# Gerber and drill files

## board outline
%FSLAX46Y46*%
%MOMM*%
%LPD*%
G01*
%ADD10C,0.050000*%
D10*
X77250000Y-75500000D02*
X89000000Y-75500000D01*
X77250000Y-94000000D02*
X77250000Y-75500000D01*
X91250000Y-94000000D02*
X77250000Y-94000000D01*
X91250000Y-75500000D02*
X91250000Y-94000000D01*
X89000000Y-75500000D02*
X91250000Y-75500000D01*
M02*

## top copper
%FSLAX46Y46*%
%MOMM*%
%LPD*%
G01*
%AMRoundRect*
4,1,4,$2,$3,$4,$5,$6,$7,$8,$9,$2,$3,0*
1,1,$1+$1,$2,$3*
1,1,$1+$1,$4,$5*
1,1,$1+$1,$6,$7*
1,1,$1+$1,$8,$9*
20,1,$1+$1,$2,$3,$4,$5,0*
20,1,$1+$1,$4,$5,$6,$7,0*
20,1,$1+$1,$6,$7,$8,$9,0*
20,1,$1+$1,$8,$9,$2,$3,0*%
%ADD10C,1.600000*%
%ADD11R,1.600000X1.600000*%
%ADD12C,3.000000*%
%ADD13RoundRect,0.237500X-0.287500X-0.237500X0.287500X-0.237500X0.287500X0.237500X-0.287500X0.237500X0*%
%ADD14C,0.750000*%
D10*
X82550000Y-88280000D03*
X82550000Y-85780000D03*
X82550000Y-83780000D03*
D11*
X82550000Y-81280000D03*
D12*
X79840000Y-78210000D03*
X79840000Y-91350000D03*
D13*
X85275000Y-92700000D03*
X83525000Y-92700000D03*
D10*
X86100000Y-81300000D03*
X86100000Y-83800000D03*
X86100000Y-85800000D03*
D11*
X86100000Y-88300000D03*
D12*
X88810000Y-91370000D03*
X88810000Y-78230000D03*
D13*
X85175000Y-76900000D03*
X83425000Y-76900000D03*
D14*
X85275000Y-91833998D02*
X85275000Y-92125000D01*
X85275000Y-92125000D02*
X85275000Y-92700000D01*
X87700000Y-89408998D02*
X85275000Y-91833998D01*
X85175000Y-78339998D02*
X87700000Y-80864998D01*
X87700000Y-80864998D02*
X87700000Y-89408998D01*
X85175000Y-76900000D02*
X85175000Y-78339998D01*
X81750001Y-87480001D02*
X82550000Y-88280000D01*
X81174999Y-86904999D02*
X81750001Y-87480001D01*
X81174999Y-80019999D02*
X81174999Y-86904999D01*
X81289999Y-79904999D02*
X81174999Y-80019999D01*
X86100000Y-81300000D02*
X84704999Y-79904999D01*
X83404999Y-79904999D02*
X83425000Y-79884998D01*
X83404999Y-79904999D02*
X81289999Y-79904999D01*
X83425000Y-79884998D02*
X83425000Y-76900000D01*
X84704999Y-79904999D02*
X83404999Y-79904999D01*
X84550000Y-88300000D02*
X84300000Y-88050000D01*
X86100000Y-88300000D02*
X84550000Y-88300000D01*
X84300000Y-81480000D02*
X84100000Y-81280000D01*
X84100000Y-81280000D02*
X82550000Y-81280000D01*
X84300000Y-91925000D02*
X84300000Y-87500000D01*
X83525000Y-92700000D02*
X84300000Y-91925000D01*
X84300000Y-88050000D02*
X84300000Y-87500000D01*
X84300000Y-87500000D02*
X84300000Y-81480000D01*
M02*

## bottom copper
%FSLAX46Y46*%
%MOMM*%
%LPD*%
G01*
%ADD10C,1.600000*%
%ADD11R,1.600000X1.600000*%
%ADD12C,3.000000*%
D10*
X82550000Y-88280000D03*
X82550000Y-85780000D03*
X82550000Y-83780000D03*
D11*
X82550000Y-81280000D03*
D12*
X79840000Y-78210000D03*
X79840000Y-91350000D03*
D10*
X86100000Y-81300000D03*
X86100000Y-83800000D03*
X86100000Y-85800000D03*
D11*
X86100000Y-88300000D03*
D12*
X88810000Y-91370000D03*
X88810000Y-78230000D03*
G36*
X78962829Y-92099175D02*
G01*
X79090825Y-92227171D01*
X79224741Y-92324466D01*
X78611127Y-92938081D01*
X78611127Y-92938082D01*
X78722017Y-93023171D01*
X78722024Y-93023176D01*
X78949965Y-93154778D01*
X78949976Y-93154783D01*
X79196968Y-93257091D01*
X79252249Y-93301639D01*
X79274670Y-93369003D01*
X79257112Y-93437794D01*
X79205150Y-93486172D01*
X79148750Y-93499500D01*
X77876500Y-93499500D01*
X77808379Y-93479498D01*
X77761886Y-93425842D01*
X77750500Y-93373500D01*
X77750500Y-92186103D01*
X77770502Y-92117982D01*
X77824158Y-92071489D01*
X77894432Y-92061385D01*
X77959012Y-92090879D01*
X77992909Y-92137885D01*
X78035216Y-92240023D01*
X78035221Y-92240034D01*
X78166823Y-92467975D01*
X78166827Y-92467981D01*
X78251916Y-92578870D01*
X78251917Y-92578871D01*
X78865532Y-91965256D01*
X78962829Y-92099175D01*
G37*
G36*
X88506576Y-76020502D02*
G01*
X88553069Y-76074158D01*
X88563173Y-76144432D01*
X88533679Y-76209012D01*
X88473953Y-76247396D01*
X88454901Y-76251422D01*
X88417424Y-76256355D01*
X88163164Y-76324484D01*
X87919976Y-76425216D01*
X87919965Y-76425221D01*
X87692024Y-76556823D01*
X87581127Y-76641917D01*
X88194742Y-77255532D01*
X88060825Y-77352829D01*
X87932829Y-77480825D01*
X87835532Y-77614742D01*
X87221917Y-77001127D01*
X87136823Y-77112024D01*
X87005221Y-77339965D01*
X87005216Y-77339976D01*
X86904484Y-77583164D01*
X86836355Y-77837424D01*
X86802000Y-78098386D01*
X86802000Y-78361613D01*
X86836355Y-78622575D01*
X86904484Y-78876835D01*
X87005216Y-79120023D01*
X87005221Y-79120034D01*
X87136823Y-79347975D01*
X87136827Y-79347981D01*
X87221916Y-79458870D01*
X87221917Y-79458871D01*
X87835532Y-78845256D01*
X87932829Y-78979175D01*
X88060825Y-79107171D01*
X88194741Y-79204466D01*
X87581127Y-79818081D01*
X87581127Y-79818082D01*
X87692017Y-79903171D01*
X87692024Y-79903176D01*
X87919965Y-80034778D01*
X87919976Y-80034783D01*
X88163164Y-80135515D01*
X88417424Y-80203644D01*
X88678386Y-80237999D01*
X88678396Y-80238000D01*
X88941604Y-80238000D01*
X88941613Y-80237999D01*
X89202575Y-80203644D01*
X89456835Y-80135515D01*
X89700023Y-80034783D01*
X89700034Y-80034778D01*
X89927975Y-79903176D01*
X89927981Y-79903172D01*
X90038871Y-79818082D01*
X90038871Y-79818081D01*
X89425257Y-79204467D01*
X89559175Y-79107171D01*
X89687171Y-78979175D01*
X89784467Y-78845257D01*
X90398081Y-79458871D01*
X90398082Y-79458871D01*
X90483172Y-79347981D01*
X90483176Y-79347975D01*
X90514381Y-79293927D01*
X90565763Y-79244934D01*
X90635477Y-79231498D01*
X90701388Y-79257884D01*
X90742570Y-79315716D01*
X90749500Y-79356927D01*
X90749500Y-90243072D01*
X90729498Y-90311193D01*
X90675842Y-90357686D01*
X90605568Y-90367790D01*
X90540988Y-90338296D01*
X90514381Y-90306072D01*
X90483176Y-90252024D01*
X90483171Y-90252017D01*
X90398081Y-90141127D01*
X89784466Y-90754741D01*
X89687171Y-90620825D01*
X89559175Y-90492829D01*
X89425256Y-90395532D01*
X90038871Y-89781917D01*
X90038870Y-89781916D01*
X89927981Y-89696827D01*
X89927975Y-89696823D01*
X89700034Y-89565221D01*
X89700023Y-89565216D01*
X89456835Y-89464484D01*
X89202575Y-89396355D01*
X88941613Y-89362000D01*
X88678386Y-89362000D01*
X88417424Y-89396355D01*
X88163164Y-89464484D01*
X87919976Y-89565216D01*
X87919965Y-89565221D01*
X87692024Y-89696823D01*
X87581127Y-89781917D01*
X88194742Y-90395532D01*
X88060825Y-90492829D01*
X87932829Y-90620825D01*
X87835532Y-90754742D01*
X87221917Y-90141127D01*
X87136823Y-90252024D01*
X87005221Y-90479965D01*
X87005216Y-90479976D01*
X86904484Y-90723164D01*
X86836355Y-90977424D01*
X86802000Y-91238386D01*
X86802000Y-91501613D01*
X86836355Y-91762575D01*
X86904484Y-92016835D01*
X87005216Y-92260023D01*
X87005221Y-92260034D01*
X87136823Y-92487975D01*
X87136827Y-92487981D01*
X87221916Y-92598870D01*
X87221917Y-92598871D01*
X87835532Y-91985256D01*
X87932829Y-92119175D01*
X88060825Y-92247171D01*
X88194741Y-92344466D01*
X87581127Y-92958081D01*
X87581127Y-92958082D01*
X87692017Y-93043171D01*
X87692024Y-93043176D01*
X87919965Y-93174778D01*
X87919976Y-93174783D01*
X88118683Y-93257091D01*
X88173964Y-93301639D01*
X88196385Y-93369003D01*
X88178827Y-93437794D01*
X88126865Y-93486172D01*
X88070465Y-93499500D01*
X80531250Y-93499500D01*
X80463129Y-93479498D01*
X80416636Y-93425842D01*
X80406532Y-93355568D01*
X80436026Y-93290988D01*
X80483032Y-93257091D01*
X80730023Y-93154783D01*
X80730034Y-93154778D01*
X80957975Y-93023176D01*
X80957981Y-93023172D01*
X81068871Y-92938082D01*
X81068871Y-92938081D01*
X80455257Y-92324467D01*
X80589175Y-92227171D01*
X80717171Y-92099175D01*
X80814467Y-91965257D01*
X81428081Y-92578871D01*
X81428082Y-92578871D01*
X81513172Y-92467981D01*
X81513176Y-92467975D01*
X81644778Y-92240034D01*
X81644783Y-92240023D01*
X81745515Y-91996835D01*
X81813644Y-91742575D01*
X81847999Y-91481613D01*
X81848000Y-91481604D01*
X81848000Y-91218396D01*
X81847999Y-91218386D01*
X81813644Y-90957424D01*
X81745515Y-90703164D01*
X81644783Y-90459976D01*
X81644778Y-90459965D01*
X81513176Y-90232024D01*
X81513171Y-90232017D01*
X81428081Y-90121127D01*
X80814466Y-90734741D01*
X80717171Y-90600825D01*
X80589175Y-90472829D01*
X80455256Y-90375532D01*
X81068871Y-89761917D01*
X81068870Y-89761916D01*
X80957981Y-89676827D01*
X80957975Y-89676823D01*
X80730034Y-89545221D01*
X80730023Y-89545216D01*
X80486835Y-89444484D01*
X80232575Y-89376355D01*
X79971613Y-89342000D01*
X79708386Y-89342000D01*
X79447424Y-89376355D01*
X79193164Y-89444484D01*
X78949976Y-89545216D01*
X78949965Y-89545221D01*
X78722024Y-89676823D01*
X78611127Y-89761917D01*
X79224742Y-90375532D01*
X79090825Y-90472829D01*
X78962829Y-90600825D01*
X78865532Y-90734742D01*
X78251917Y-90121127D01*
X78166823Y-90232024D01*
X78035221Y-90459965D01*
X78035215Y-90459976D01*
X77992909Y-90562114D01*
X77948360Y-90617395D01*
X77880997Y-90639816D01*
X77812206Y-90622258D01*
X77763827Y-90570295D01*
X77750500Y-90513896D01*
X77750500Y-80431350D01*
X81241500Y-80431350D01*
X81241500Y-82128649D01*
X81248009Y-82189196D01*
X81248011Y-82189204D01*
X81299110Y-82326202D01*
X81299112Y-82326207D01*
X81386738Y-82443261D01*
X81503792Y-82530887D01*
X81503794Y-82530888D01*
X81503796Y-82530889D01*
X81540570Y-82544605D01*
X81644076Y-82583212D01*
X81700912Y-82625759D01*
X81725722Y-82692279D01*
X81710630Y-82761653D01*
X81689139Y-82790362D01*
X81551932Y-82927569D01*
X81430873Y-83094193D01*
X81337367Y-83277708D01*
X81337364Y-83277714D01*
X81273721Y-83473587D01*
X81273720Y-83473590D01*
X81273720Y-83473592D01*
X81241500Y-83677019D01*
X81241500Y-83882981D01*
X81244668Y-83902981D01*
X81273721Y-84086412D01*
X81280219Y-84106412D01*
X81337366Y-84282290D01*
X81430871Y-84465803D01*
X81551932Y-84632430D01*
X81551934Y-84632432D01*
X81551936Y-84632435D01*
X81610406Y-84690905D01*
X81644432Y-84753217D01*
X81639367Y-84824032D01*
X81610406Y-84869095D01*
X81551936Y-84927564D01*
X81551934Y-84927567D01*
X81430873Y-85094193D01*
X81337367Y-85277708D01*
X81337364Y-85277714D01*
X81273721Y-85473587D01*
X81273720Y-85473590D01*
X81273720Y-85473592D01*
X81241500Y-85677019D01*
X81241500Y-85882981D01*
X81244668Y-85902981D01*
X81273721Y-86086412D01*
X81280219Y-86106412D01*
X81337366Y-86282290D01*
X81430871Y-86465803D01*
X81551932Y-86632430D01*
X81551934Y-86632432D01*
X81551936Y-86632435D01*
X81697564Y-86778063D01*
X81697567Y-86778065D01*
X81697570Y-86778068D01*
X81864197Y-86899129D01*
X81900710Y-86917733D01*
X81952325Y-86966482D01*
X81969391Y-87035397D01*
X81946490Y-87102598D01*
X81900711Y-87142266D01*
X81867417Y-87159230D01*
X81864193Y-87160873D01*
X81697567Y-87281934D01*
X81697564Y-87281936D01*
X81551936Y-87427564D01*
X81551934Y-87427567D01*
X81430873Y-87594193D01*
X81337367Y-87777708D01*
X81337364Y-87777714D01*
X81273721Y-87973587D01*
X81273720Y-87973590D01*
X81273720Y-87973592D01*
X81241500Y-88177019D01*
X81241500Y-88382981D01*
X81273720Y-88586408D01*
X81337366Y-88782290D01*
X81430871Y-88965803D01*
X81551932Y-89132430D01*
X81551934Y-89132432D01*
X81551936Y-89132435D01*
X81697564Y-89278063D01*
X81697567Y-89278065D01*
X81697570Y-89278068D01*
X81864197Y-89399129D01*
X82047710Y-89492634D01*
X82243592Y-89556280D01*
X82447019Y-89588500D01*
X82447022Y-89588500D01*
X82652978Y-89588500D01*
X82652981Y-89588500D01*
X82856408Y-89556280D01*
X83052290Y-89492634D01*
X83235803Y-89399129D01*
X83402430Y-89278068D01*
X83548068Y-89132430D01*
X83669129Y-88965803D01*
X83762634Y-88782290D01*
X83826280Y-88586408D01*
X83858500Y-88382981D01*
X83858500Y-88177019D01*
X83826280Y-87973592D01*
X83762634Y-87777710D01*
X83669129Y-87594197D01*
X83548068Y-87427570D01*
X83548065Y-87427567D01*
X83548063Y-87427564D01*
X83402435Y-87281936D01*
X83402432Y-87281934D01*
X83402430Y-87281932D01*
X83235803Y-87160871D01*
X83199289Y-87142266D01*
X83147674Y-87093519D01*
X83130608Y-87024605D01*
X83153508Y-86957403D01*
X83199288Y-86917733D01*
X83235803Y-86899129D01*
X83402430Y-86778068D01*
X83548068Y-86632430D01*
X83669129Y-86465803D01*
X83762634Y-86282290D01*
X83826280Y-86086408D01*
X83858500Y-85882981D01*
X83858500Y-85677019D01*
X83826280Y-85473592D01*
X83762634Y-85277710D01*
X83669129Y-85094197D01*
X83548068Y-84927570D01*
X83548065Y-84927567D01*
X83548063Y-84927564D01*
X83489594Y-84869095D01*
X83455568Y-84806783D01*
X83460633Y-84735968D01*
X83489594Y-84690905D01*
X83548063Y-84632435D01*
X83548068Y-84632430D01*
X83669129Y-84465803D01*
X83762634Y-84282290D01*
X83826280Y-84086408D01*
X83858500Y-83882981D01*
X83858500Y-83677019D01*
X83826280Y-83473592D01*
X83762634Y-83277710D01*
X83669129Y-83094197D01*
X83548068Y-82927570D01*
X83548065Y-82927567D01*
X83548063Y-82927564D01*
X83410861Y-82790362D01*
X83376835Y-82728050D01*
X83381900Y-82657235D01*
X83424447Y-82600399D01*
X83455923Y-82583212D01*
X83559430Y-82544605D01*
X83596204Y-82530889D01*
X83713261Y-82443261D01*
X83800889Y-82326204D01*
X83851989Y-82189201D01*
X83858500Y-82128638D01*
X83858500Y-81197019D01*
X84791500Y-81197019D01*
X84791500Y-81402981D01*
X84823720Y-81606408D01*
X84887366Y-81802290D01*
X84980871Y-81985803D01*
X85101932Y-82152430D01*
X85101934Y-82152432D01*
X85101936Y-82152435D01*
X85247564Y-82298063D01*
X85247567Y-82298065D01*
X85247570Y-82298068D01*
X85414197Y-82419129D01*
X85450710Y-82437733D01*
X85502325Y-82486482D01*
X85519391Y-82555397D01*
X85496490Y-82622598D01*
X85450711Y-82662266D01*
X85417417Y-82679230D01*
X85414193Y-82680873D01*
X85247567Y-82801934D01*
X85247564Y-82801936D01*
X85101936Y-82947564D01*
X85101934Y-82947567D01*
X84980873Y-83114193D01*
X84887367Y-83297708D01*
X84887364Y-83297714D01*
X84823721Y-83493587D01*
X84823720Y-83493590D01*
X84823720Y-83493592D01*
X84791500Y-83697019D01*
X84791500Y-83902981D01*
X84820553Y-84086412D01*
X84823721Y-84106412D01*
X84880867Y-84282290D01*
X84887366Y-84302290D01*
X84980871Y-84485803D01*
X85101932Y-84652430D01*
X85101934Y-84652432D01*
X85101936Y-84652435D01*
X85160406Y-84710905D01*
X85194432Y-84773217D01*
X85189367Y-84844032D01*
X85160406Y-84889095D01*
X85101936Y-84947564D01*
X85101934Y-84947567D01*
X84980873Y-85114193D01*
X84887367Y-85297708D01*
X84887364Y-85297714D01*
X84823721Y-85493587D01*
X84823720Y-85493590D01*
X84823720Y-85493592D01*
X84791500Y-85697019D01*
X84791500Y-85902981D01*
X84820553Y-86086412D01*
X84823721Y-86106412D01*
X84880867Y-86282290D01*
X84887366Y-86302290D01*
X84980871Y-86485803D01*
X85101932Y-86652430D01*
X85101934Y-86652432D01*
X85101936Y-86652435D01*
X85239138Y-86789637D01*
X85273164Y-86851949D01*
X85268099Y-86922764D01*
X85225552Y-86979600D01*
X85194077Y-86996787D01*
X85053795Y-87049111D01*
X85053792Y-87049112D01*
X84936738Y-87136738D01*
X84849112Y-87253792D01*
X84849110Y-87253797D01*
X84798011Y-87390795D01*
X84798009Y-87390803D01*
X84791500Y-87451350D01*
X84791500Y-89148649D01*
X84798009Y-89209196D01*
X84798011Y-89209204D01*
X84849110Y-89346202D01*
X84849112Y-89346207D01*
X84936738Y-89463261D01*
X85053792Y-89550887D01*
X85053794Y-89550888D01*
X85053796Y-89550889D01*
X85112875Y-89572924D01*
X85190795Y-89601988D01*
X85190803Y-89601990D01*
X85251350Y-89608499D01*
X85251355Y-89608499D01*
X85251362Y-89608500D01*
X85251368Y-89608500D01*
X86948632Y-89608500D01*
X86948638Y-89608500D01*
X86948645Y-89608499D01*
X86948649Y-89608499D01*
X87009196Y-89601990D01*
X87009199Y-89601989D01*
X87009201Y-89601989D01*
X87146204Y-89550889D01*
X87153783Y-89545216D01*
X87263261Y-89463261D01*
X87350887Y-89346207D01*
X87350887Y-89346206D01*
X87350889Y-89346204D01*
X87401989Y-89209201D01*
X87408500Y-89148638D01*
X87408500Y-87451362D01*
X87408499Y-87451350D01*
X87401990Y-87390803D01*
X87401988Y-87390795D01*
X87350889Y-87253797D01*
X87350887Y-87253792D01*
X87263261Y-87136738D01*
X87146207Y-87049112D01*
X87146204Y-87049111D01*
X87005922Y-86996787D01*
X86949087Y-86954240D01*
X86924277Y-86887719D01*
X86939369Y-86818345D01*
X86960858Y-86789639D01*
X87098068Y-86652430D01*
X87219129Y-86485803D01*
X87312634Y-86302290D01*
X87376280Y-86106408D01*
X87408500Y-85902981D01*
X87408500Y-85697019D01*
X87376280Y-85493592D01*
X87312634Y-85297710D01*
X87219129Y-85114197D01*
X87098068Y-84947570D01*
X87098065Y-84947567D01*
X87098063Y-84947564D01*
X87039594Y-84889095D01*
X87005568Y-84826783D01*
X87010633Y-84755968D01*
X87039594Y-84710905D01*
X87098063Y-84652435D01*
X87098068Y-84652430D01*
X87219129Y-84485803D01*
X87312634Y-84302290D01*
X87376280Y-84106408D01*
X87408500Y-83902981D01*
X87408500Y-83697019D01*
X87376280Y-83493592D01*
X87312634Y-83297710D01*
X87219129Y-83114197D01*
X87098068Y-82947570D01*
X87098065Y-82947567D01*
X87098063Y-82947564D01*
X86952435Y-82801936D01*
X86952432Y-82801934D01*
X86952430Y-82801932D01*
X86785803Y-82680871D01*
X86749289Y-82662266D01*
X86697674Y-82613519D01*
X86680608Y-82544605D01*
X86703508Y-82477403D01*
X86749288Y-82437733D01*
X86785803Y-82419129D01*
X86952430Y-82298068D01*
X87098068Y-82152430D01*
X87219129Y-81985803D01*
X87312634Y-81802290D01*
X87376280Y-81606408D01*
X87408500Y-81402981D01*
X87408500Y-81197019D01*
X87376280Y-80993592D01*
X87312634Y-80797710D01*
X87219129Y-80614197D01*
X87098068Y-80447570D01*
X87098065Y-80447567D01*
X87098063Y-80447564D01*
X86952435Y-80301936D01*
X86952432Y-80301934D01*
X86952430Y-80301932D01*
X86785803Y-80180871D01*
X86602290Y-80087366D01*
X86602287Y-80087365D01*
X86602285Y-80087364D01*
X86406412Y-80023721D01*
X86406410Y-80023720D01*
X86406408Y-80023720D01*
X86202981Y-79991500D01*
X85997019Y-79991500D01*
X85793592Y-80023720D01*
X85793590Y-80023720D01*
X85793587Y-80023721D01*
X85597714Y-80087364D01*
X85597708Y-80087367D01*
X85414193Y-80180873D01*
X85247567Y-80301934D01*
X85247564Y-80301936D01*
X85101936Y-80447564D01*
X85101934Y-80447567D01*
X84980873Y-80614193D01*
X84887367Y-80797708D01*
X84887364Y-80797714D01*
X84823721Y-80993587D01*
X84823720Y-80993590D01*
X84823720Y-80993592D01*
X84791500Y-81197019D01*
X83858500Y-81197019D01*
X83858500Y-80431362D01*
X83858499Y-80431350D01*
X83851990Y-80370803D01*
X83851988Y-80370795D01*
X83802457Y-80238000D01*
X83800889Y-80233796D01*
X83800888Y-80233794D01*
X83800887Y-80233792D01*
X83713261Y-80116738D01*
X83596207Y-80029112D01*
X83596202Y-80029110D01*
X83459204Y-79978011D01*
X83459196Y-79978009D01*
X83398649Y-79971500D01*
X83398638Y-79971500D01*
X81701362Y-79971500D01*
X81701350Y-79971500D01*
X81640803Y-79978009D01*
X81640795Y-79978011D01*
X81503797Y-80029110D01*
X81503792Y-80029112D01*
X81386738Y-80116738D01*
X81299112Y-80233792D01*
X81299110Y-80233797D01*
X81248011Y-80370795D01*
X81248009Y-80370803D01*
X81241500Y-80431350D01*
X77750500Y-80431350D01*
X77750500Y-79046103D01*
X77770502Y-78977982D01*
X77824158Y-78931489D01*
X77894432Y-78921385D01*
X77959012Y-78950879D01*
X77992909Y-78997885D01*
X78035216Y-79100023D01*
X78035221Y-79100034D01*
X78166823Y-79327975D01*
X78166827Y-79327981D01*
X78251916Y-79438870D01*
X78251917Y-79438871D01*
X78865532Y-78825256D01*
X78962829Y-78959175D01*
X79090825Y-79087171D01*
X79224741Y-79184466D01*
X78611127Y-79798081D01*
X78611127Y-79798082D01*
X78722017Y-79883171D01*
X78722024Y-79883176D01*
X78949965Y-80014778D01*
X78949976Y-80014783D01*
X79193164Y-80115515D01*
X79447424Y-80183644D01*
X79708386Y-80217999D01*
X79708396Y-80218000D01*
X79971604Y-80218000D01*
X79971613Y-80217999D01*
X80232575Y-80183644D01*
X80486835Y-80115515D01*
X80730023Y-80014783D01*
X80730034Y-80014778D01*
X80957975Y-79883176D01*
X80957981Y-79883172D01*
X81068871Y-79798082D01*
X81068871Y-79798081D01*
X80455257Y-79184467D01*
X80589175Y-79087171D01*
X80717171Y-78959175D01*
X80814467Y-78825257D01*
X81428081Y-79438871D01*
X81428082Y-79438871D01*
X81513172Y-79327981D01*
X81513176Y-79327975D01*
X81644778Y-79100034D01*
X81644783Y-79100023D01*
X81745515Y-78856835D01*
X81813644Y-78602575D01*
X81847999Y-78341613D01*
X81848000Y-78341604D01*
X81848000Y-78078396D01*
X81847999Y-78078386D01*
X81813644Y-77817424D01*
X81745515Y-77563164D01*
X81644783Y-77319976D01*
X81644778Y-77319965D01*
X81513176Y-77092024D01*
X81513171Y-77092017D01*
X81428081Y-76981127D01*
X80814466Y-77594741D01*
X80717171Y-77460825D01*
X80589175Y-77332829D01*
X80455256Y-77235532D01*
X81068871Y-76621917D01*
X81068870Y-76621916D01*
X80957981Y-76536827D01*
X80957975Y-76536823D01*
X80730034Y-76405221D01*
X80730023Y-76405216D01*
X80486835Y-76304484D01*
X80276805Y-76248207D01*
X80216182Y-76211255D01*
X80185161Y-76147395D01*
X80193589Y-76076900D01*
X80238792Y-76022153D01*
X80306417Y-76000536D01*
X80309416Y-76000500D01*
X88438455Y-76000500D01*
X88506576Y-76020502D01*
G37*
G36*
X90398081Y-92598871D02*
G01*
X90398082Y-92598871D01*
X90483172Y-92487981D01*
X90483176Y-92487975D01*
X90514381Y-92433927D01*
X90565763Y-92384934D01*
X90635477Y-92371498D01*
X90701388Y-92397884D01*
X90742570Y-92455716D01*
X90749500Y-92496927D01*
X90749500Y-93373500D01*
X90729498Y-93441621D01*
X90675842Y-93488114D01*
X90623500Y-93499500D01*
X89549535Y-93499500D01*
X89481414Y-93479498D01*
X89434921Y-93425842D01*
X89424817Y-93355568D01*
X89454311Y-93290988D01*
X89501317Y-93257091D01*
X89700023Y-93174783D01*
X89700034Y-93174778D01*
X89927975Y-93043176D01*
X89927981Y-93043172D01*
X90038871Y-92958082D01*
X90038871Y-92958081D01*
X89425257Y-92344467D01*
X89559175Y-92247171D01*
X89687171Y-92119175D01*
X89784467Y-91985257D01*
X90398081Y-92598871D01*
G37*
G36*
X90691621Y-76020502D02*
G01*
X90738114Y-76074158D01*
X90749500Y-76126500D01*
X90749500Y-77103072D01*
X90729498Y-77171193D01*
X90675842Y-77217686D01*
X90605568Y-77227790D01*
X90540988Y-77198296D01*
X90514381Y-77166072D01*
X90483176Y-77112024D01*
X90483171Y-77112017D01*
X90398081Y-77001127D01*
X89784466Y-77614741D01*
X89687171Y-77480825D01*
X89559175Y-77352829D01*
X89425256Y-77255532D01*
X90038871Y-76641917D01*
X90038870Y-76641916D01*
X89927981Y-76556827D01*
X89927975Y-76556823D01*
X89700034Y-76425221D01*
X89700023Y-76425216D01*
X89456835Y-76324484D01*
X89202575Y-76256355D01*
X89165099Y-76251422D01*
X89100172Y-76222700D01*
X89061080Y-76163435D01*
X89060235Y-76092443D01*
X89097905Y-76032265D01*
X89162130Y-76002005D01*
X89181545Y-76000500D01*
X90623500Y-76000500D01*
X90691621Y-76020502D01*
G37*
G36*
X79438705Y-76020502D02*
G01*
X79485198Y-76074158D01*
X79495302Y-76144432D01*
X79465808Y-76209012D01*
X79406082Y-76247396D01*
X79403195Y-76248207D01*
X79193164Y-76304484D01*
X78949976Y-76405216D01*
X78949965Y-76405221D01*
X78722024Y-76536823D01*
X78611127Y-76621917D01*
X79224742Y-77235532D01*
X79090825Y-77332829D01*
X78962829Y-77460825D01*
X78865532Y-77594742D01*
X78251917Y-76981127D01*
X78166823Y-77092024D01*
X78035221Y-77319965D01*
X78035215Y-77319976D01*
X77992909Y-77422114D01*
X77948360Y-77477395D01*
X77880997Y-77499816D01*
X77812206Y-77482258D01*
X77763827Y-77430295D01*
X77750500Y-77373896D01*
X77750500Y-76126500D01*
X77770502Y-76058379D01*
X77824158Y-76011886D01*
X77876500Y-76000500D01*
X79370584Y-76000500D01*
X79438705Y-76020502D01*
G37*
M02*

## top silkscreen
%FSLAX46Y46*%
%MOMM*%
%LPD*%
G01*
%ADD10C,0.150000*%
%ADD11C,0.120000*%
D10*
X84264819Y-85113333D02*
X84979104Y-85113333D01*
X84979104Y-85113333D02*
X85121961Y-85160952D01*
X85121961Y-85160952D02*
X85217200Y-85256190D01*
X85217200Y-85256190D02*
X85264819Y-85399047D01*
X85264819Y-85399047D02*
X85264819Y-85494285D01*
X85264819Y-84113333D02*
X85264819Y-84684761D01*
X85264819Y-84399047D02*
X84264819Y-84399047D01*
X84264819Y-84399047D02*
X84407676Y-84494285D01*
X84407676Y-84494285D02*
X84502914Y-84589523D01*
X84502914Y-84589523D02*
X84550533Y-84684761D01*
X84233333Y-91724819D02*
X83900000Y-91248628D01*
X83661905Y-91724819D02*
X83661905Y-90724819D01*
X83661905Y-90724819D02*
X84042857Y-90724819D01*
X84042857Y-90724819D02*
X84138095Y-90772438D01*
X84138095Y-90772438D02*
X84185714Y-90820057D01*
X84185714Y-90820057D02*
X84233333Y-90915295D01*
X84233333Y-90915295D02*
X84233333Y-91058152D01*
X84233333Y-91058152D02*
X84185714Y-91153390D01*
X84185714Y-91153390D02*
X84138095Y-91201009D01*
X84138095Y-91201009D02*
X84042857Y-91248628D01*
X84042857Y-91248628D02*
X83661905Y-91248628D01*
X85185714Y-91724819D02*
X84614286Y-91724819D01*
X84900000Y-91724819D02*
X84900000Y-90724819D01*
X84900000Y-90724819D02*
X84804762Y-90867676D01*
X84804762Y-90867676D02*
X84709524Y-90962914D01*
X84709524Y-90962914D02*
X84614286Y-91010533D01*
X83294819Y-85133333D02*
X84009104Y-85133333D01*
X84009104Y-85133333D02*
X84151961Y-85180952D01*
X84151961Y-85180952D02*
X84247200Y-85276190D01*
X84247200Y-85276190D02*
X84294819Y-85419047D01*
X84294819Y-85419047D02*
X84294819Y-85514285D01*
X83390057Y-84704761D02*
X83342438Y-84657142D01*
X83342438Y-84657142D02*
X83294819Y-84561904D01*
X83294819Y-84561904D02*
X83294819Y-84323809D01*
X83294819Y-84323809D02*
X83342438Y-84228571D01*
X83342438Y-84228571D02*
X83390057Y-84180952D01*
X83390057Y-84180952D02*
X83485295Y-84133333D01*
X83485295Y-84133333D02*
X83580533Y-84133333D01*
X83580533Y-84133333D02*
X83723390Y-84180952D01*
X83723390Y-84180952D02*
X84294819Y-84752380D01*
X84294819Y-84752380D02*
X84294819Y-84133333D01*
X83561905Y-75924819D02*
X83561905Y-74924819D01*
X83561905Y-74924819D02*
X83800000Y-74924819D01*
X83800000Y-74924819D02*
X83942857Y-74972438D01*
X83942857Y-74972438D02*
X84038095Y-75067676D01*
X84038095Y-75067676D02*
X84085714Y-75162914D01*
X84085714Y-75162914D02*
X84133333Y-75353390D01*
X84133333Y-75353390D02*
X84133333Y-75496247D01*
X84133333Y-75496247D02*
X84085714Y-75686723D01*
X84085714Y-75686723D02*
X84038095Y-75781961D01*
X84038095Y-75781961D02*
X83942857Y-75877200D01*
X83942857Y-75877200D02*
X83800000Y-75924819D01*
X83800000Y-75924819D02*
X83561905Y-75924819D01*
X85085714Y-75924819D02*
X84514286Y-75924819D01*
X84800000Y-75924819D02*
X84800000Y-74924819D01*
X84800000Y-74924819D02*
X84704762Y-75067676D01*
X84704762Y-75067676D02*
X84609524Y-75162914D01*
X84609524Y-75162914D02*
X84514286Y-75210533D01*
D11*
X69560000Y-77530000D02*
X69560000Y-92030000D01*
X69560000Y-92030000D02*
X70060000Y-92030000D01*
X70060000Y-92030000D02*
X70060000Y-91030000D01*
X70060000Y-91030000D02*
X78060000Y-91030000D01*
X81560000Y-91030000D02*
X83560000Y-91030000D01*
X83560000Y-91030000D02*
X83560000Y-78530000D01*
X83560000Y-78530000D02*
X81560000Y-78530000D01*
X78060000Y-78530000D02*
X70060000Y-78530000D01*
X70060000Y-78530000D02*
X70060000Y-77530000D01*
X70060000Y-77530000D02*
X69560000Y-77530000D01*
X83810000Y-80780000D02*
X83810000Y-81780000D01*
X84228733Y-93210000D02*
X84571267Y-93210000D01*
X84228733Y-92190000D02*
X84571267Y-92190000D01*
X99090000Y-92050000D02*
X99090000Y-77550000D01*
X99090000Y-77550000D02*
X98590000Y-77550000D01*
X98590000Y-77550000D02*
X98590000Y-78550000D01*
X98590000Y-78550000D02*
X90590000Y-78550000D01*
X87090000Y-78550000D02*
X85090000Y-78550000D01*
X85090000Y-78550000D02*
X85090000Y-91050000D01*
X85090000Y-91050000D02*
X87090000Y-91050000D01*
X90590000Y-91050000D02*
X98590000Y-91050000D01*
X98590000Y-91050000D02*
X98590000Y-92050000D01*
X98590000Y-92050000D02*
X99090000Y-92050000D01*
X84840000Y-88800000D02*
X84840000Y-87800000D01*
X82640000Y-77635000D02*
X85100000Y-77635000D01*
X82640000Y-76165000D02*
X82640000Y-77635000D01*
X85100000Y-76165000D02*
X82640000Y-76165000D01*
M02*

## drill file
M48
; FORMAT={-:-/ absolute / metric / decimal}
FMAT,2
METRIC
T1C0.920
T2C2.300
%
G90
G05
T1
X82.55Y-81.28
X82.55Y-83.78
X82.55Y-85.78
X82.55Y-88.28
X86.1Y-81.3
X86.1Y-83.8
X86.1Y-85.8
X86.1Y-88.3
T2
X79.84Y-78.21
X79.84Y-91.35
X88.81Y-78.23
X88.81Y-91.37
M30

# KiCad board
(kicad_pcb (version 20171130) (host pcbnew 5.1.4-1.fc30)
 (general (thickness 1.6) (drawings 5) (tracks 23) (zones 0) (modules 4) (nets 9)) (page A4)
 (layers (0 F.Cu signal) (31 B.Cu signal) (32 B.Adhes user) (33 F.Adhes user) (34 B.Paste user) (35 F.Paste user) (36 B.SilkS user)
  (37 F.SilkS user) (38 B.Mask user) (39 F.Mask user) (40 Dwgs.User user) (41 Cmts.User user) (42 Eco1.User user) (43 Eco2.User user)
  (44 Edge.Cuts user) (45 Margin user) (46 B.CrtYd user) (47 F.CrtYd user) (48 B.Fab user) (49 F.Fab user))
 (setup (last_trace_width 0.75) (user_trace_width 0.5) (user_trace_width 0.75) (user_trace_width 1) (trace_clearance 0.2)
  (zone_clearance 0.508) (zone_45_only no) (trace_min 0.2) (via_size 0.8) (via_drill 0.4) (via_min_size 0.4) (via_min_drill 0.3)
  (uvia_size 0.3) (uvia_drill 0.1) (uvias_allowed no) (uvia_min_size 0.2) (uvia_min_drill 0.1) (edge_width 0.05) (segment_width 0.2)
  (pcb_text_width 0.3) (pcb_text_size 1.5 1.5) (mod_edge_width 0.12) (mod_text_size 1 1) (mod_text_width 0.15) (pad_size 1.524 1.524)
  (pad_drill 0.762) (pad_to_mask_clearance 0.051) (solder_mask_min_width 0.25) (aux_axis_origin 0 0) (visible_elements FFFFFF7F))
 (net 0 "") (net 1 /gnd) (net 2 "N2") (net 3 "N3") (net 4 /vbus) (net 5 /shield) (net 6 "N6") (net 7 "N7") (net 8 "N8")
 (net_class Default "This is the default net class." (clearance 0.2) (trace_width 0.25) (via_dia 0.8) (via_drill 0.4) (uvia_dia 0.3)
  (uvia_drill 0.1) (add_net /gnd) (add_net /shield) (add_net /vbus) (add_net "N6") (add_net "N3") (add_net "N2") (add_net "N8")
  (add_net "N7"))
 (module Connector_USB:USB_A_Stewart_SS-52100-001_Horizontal (layer F.Cu) (at 82.55 81.28 270)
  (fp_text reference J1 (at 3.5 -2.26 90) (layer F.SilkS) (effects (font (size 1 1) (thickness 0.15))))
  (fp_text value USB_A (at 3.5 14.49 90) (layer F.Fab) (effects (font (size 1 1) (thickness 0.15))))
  (fp_line (start -3.75 12.99) (end 10.75 12.99) (layer F.SilkS) (width 0.12))
  (fp_line (start 10.75 12.99) (end 10.75 12.49) (layer F.SilkS) (width 0.12))
  (fp_line (start 10.75 12.49) (end 9.75 12.49) (layer F.SilkS) (width 0.12))
  (fp_line (start 9.75 12.49) (end 9.75 4.49) (layer F.SilkS) (width 0.12))
  (fp_line (start 9.75 0.99) (end 9.75 -1.01) (layer F.SilkS) (width 0.12))
  (fp_line (start 9.75 -1.01) (end -2.75 -1.01) (layer F.SilkS) (width 0.12))
  (fp_line (start -2.75 -1.01) (end -2.75 0.99) (layer F.SilkS) (width 0.12))
  (fp_line (start -2.75 4.49) (end -2.75 12.49) (layer F.SilkS) (width 0.12))
  (fp_line (start -2.75 12.49) (end -3.75 12.49) (layer F.SilkS) (width 0.12))
  (fp_line (start -3.75 12.49) (end -3.75 12.99) (layer F.SilkS) (width 0.12))
  (fp_line (start -0.5 -1.26) (end 0.5 -1.26) (layer F.SilkS) (width 0.12))
  (pad 4 thru_hole circle (at 7 0 270) (size 1.6 1.6) (drill 0.92) (layers *.Cu *.Mask) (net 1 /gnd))
  (pad 3 thru_hole circle (at 4.5 0 270) (size 1.6 1.6) (drill 0.92) (layers *.Cu *.Mask) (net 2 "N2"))
  (pad 2 thru_hole circle (at 2.5 0 270) (size 1.6 1.6) (drill 0.92) (layers *.Cu *.Mask) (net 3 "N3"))
  (pad 1 thru_hole rect (at 0 0 270) (size 1.6 1.6) (drill 0.92) (layers *.Cu *.Mask) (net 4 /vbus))
  (pad 5 thru_hole circle (at -3.07 2.71 270) (size 3 3) (drill 2.3) (layers *.Cu *.Mask) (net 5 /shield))
  (pad 5 thru_hole circle (at 10.07 2.71 270) (size 3 3) (drill 2.3) (layers *.Cu *.Mask) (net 5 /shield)))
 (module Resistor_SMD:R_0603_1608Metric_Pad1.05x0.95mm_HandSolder (layer F.Cu) (at 84.4 92.7)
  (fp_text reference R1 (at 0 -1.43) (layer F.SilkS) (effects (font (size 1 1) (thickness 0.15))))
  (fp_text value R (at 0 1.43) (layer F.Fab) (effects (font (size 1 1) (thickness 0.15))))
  (fp_line (start -0.171267 0.51) (end 0.171267 0.51) (layer F.SilkS) (width 0.12))
  (fp_line (start -0.171267 -0.51) (end 0.171267 -0.51) (layer F.SilkS) (width 0.12))
  (pad 2 smd roundrect (at 0.875 0) (size 1.05 0.95) (layers F.Cu F.Paste F.Mask) (roundrect_rratio 0.25) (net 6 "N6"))
  (pad 1 smd roundrect (at -0.875 0) (size 1.05 0.95) (layers F.Cu F.Paste F.Mask) (roundrect_rratio 0.25) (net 4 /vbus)))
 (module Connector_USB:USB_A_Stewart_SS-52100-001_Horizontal (layer F.Cu) (at 86.1 88.3 90)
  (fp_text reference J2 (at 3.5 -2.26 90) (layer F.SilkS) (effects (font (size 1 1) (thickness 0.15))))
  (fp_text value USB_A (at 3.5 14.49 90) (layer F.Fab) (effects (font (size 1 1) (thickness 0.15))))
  (fp_line (start -3.75 12.99) (end 10.75 12.99) (layer F.SilkS) (width 0.12))
  (fp_line (start 10.75 12.99) (end 10.75 12.49) (layer F.SilkS) (width 0.12))
  (fp_line (start 10.75 12.49) (end 9.75 12.49) (layer F.SilkS) (width 0.12))
  (fp_line (start 9.75 12.49) (end 9.75 4.49) (layer F.SilkS) (width 0.12))
  (fp_line (start 9.75 0.99) (end 9.75 -1.01) (layer F.SilkS) (width 0.12))
  (fp_line (start 9.75 -1.01) (end -2.75 -1.01) (layer F.SilkS) (width 0.12))
  (fp_line (start -2.75 -1.01) (end -2.75 0.99) (layer F.SilkS) (width 0.12))
  (fp_line (start -2.75 4.49) (end -2.75 12.49) (layer F.SilkS) (width 0.12))
  (fp_line (start -2.75 12.49) (end -3.75 12.49) (layer F.SilkS) (width 0.12))
  (fp_line (start -3.75 12.49) (end -3.75 12.99) (layer F.SilkS) (width 0.12))
  (fp_line (start -0.5 -1.26) (end 0.5 -1.26) (layer F.SilkS) (width 0.12))
  (pad 4 thru_hole circle (at 7 0 90) (size 1.6 1.6) (drill 0.92) (layers *.Cu *.Mask) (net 1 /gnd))
  (pad 3 thru_hole circle (at 4.5 0 90) (size 1.6 1.6) (drill 0.92) (layers *.Cu *.Mask) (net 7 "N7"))
  (pad 2 thru_hole circle (at 2.5 0 90) (size 1.6 1.6) (drill 0.92) (layers *.Cu *.Mask) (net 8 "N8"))
  (pad 1 thru_hole rect (at 0 0 90) (size 1.6 1.6) (drill 0.92) (layers *.Cu *.Mask) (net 4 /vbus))
  (pad 5 thru_hole circle (at -3.07 2.71 90) (size 3 3) (drill 2.3) (layers *.Cu *.Mask) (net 5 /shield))
  (pad 5 thru_hole circle (at 10.07 2.71 90) (size 3 3) (drill 2.3) (layers *.Cu *.Mask) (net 5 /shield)))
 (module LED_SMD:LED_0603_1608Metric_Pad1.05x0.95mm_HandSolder (layer F.Cu) (at 84.3 76.9)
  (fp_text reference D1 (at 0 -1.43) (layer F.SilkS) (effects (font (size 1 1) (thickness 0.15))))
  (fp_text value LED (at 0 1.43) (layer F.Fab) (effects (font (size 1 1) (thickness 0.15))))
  (fp_line (start -1.66 0.735) (end 0.8 0.735) (layer F.SilkS) (width 0.12))
  (fp_line (start -1.66 -0.735) (end -1.66 0.735) (layer F.SilkS) (width 0.12))
  (fp_line (start 0.8 -0.735) (end -1.66 -0.735) (layer F.SilkS) (width 0.12))
  (pad 2 smd roundrect (at 0.875 0) (size 1.05 0.95) (layers F.Cu F.Paste F.Mask) (roundrect_rratio 0.25) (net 6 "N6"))
  (pad 1 smd roundrect (at -0.875 0) (size 1.05 0.95) (layers F.Cu F.Paste F.Mask) (roundrect_rratio 0.25) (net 1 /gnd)))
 (gr_line (start 77.25 75.5) (end 89 75.5) (layer Edge.Cuts) (width 0.05))
 (gr_line (start 77.25 94) (end 77.25 75.5) (layer Edge.Cuts) (width 0.05))
 (gr_line (start 91.25 94) (end 77.25 94) (layer Edge.Cuts) (width 0.05))
 (gr_line (start 91.25 75.5) (end 91.25 94) (layer Edge.Cuts) (width 0.05))
 (gr_line (start 89 75.5) (end 91.25 75.5) (layer Edge.Cuts) (width 0.05))
 (segment (start 85.275 91.833998) (end 85.275 92.125) (width 0.75) (layer F.Cu) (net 6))
 (segment (start 85.275 92.125) (end 85.275 92.7) (width 0.75) (layer F.Cu) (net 6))
 (segment (start 87.7 89.408998) (end 85.275 91.833998) (width 0.75) (layer F.Cu) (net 6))
 (segment (start 85.175 78.339998) (end 87.7 80.864998) (width 0.75) (layer F.Cu) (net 6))
 (segment (start 87.7 80.864998) (end 87.7 89.408998) (width 0.75) (layer F.Cu) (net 6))
 (segment (start 85.175 76.9) (end 85.175 78.339998) (width 0.75) (layer F.Cu) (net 6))
 (segment (start 81.750001 87.480001) (end 82.55 88.28) (width 0.75) (layer F.Cu) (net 1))
 (segment (start 81.174999 86.904999) (end 81.750001 87.480001) (width 0.75) (layer F.Cu) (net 1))
 (segment (start 81.174999 80.019999) (end 81.174999 86.904999) (width 0.75) (layer F.Cu) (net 1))
 (segment (start 81.289999 79.904999) (end 81.174999 80.019999) (width 0.75) (layer F.Cu) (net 1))
 (segment (start 86.1 81.3) (end 84.704999 79.904999) (width 0.75) (layer F.Cu) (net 1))
 (segment (start 83.404999 79.904999) (end 83.425 79.884998) (width 0.75) (layer F.Cu) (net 1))
 (segment (start 83.404999 79.904999) (end 81.289999 79.904999) (width 0.75) (layer F.Cu) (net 1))
 (segment (start 83.425 79.884998) (end 83.425 76.9) (width 0.75) (layer F.Cu) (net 1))
 (segment (start 84.704999 79.904999) (end 83.404999 79.904999) (width 0.75) (layer F.Cu) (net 1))
 (segment (start 84.55 88.3) (end 84.3 88.05) (width 0.75) (layer F.Cu) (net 4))
 (segment (start 86.1 88.3) (end 84.55 88.3) (width 0.75) (layer F.Cu) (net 4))
 (segment (start 84.3 81.48) (end 84.1 81.28) (width 0.75) (layer F.Cu) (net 4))
 (segment (start 84.1 81.28) (end 82.55 81.28) (width 0.75) (layer F.Cu) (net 4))
 (segment (start 84.3 91.925) (end 84.3 87.5) (width 0.75) (layer F.Cu) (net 4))
 (segment (start 83.525 92.7) (end 84.3 91.925) (width 0.75) (layer F.Cu) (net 4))
 (segment (start 84.3 88.05) (end 84.3 87.5) (width 0.75) (layer F.Cu) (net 4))
 (segment (start 84.3 87.5) (end 84.3 81.48) (width 0.75) (layer F.Cu) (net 4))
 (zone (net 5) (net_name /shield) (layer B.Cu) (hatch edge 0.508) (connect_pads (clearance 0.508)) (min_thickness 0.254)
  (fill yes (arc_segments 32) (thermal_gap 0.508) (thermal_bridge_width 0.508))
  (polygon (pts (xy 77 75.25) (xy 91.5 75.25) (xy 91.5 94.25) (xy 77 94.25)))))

